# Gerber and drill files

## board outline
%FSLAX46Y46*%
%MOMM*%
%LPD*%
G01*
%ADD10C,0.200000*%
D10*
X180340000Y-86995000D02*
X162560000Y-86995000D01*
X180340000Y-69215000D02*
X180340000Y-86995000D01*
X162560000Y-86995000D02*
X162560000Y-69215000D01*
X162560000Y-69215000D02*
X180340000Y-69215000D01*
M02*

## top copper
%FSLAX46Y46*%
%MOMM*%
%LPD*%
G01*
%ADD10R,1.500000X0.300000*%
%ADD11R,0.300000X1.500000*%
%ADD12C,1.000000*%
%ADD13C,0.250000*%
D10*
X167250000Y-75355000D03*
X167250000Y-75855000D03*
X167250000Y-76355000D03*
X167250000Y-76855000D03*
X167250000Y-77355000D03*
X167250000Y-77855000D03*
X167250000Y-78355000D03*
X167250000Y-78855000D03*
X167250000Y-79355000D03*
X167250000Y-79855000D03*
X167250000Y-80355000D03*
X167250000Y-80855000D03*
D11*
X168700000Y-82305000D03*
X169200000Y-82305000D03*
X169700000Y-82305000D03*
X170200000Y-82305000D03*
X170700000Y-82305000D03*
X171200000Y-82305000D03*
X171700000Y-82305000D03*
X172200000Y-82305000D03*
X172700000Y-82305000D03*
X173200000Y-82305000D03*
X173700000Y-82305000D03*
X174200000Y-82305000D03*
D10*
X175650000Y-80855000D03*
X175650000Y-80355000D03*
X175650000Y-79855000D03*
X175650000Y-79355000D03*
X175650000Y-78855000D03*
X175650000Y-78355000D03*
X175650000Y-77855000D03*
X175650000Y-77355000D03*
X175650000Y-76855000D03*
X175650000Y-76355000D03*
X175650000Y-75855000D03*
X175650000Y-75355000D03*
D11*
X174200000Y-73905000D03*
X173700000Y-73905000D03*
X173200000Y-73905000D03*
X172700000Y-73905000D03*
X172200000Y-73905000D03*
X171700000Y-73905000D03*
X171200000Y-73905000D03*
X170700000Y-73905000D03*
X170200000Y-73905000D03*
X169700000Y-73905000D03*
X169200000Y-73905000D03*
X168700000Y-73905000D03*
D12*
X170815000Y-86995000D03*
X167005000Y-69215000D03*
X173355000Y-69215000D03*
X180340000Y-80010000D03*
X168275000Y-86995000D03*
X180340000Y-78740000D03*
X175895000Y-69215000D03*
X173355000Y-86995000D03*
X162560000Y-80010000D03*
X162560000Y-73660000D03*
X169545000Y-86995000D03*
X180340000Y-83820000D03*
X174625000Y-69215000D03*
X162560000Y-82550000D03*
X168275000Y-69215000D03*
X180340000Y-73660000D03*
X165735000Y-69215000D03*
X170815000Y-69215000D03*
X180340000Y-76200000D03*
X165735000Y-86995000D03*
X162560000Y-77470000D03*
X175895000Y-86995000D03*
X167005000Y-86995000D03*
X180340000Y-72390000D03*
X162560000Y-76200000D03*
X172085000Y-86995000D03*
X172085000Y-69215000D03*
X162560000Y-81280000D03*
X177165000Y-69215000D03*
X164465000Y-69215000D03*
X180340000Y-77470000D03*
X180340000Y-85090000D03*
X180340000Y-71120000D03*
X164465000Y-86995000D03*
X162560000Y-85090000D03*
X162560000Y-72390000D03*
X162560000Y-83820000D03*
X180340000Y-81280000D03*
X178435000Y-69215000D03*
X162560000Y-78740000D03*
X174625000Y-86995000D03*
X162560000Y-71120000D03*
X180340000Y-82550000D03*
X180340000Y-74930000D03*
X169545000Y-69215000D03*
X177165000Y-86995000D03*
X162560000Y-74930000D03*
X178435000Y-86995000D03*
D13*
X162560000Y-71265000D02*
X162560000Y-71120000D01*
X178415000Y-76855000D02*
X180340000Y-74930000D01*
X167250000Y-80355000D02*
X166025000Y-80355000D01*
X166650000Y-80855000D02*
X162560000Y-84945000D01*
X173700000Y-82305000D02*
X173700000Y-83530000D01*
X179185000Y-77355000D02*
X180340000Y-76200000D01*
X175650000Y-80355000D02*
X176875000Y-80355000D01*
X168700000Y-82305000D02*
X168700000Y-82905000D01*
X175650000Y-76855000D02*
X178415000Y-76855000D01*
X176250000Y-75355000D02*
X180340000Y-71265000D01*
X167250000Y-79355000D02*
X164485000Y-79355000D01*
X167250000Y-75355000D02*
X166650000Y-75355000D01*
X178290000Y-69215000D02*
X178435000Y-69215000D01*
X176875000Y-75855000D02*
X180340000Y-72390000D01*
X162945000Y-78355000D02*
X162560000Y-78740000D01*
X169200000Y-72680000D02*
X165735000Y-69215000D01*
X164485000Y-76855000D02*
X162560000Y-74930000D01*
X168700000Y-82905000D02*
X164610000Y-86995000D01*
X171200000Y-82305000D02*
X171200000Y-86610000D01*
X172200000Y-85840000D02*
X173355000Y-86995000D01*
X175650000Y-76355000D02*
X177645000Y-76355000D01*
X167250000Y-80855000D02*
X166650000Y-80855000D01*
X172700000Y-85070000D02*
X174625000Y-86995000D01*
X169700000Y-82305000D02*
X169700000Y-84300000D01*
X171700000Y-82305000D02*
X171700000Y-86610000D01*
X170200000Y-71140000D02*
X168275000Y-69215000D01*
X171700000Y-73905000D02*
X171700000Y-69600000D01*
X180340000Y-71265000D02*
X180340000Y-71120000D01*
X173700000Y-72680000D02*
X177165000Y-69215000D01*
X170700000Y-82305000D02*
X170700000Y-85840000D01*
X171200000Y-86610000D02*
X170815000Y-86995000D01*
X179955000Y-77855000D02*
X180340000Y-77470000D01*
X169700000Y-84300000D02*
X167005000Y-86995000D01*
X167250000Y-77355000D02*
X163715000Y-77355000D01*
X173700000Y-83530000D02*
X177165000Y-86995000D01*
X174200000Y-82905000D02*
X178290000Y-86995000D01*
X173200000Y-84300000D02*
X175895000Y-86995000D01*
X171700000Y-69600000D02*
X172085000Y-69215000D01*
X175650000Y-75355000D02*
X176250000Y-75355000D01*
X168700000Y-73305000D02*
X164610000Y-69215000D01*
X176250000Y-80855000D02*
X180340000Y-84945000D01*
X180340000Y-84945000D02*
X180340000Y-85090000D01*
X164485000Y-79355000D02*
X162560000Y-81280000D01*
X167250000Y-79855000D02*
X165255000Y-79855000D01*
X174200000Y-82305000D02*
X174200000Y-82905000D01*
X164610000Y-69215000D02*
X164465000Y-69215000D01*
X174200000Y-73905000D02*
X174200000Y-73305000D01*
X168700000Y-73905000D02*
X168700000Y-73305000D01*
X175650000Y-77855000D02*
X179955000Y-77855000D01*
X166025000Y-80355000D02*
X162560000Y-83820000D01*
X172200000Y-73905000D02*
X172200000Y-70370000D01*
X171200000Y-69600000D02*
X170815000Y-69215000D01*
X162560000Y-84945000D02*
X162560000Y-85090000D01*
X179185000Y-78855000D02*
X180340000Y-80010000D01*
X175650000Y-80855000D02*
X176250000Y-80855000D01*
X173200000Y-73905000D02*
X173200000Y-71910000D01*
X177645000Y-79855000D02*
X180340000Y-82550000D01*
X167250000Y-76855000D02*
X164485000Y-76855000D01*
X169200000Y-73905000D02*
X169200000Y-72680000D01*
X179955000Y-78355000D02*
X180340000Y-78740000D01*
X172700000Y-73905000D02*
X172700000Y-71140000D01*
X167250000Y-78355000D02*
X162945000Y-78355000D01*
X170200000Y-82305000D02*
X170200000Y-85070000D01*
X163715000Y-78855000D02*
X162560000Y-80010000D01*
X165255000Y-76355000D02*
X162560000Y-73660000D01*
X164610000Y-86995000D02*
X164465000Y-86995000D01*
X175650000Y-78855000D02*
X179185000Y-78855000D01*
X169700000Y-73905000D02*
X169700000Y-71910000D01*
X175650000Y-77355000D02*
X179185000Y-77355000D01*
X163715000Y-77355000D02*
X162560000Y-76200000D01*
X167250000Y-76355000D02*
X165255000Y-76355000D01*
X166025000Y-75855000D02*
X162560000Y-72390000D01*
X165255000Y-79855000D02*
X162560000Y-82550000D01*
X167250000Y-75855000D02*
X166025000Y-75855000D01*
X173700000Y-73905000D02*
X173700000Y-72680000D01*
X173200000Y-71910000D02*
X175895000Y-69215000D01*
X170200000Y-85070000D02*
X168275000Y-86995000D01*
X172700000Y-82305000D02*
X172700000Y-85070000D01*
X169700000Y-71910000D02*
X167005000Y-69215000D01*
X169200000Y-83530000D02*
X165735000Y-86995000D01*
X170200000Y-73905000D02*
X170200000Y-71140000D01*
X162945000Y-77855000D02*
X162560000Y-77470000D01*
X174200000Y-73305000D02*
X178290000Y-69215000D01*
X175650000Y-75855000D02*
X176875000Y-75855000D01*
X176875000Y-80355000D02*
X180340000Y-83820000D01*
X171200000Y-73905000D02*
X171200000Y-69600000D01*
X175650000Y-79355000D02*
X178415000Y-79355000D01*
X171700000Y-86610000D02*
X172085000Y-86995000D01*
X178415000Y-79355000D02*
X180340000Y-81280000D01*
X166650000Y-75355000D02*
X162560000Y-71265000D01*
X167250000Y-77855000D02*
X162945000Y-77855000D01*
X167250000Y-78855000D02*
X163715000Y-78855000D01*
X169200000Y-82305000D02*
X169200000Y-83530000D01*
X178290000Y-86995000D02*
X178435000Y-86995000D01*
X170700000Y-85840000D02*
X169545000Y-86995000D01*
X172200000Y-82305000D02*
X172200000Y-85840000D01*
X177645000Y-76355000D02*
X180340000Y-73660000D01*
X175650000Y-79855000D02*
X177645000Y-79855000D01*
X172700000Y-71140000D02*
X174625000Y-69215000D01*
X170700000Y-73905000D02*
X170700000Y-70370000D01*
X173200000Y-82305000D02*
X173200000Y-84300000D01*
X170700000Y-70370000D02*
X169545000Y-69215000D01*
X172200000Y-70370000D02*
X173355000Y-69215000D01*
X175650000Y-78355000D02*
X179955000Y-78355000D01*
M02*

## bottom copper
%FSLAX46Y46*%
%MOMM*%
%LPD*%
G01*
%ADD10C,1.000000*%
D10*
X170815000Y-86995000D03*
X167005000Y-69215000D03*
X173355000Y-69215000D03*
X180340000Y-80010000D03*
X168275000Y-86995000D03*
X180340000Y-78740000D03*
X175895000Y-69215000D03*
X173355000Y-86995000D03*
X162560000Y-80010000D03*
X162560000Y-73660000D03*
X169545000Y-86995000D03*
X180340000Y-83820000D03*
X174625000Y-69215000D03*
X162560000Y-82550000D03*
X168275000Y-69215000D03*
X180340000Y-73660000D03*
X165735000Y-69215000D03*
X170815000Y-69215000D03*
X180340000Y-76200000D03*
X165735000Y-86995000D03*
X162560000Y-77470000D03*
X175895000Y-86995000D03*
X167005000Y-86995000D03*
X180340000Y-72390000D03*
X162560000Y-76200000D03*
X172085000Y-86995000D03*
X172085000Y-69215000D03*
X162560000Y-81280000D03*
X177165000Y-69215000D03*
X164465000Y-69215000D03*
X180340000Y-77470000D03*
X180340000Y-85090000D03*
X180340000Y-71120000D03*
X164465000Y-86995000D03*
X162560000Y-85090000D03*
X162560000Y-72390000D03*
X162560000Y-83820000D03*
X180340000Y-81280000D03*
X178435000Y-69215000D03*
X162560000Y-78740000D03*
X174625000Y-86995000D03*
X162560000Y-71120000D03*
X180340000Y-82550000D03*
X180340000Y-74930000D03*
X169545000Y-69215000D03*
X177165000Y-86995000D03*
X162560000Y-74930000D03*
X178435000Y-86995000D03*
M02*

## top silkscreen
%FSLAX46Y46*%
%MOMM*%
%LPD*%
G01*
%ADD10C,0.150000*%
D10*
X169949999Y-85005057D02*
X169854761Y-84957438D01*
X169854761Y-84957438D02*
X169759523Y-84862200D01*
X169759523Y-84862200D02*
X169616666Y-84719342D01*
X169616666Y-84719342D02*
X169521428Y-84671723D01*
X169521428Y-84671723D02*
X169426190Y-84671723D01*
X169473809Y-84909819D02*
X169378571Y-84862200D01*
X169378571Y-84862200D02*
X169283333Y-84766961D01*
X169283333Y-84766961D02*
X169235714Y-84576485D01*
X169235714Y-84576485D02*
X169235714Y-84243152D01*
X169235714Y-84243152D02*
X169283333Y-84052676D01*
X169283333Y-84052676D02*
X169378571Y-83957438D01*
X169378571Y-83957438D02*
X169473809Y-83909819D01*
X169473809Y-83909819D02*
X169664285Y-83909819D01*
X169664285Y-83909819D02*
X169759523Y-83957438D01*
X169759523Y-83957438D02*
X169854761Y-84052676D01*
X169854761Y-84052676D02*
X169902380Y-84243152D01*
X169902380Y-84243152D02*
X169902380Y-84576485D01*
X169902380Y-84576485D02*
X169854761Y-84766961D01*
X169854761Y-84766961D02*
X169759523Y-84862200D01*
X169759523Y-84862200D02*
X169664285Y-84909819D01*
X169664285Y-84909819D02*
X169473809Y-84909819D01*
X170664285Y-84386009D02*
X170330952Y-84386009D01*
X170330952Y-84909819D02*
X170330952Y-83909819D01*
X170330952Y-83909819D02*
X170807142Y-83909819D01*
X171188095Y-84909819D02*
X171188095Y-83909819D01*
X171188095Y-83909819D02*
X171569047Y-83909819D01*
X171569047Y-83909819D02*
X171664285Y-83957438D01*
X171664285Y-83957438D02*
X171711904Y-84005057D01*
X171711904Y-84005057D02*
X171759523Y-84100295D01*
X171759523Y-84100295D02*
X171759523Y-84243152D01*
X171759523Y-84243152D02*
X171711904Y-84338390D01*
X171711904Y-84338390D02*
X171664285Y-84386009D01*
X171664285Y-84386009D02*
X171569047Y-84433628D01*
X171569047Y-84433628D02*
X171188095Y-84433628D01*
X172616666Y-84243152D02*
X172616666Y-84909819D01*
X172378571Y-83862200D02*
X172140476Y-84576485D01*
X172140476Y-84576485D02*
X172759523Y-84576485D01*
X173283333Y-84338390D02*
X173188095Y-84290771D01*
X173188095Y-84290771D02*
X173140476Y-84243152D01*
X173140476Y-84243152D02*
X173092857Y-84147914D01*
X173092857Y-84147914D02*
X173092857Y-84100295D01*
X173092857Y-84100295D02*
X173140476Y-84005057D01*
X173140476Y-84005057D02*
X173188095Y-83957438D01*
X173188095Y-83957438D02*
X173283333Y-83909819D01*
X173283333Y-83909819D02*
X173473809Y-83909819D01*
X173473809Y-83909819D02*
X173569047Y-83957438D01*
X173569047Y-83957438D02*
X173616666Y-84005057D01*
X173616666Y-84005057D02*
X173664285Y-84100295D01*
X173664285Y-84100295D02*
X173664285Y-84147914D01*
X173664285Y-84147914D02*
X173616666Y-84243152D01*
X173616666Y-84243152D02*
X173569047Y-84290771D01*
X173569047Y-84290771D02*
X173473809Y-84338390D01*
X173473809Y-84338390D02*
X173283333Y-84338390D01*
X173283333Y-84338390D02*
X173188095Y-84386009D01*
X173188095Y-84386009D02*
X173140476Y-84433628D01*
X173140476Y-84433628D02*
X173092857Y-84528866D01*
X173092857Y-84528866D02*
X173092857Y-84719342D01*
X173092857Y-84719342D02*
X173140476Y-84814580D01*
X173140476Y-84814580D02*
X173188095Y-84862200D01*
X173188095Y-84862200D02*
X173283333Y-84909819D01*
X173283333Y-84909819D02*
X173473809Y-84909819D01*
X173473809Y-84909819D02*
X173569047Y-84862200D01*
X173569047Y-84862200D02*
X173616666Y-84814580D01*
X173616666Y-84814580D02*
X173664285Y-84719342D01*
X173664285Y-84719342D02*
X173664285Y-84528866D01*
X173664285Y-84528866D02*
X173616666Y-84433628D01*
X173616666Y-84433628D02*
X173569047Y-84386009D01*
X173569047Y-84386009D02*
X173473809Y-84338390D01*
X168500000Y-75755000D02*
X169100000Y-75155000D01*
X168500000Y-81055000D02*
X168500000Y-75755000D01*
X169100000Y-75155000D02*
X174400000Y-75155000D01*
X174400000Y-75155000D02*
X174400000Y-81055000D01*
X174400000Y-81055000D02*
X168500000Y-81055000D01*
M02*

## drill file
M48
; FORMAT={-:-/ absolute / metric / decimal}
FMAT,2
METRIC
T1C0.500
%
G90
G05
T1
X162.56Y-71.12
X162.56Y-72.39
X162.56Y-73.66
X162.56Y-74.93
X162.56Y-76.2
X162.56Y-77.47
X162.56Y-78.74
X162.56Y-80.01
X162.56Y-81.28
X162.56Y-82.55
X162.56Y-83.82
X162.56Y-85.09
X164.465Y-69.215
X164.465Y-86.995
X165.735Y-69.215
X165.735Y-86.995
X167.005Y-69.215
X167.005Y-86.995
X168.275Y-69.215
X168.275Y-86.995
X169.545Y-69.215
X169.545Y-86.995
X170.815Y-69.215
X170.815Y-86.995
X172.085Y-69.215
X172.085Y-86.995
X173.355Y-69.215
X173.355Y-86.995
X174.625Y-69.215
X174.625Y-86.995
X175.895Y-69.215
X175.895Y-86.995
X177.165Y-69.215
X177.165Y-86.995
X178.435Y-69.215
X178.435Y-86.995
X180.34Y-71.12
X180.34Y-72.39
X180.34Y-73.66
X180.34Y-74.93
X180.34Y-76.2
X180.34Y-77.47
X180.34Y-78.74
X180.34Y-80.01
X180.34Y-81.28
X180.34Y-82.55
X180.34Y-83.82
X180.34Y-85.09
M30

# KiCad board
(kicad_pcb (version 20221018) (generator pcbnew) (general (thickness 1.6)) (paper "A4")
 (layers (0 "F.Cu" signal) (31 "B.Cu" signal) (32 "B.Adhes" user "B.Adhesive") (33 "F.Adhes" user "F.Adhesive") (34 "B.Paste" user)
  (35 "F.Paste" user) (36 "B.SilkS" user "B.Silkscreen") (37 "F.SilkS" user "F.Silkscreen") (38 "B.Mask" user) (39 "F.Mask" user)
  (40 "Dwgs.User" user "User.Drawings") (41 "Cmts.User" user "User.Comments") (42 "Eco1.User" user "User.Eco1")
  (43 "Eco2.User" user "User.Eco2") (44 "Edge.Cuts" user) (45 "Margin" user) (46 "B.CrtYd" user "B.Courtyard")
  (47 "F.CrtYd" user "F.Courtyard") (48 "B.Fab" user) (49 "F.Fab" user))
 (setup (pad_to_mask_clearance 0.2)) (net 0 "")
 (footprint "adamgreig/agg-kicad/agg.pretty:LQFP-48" (layer "F.Cu") (at 171.45 78.105)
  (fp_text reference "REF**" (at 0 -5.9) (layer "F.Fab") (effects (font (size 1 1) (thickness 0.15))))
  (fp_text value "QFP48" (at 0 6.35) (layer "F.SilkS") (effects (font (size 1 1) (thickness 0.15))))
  (fp_line (start -2.95 -2.35) (end -2.35 -2.95) (stroke (width 0.15) (type solid)) (layer "F.SilkS"))
  (fp_line (start -2.95 2.95) (end -2.95 -2.35) (stroke (width 0.15) (type solid)) (layer "F.SilkS"))
  (fp_line (start -2.35 -2.95) (end 2.95 -2.95) (stroke (width 0.15) (type solid)) (layer "F.SilkS"))
  (fp_line (start 2.95 -2.95) (end 2.95 2.95) (stroke (width 0.15) (type solid)) (layer "F.SilkS"))
  (fp_line (start 2.95 2.95) (end -2.95 2.95) (stroke (width 0.15) (type solid)) (layer "F.SilkS"))
  (pad "1" smd rect (at -4.2 -2.75) (size 1.5 0.3) (layers "F.Cu" "F.Paste" "F.Mask"))
  (pad "2" smd rect (at -4.2 -2.25) (size 1.5 0.3) (layers "F.Cu" "F.Paste" "F.Mask"))
  (pad "3" smd rect (at -4.2 -1.75) (size 1.5 0.3) (layers "F.Cu" "F.Paste" "F.Mask"))
  (pad "4" smd rect (at -4.2 -1.25) (size 1.5 0.3) (layers "F.Cu" "F.Paste" "F.Mask"))
  (pad "5" smd rect (at -4.2 -0.75) (size 1.5 0.3) (layers "F.Cu" "F.Paste" "F.Mask"))
  (pad "6" smd rect (at -4.2 -0.25) (size 1.5 0.3) (layers "F.Cu" "F.Paste" "F.Mask"))
  (pad "7" smd rect (at -4.2 0.25) (size 1.5 0.3) (layers "F.Cu" "F.Paste" "F.Mask"))
  (pad "8" smd rect (at -4.2 0.75) (size 1.5 0.3) (layers "F.Cu" "F.Paste" "F.Mask"))
  (pad "9" smd rect (at -4.2 1.25) (size 1.5 0.3) (layers "F.Cu" "F.Paste" "F.Mask"))
  (pad "10" smd rect (at -4.2 1.75) (size 1.5 0.3) (layers "F.Cu" "F.Paste" "F.Mask"))
  (pad "11" smd rect (at -4.2 2.25) (size 1.5 0.3) (layers "F.Cu" "F.Paste" "F.Mask"))
  (pad "12" smd rect (at -4.2 2.75) (size 1.5 0.3) (layers "F.Cu" "F.Paste" "F.Mask"))
  (pad "13" smd rect (at -2.75 4.2) (size 0.3 1.5) (layers "F.Cu" "F.Paste" "F.Mask"))
  (pad "14" smd rect (at -2.25 4.2) (size 0.3 1.5) (layers "F.Cu" "F.Paste" "F.Mask"))
  (pad "15" smd rect (at -1.75 4.2) (size 0.3 1.5) (layers "F.Cu" "F.Paste" "F.Mask"))
  (pad "16" smd rect (at -1.25 4.2) (size 0.3 1.5) (layers "F.Cu" "F.Paste" "F.Mask"))
  (pad "17" smd rect (at -0.75 4.2) (size 0.3 1.5) (layers "F.Cu" "F.Paste" "F.Mask"))
  (pad "18" smd rect (at -0.25 4.2) (size 0.3 1.5) (layers "F.Cu" "F.Paste" "F.Mask"))
  (pad "19" smd rect (at 0.25 4.2) (size 0.3 1.5) (layers "F.Cu" "F.Paste" "F.Mask"))
  (pad "20" smd rect (at 0.75 4.2) (size 0.3 1.5) (layers "F.Cu" "F.Paste" "F.Mask"))
  (pad "21" smd rect (at 1.25 4.2) (size 0.3 1.5) (layers "F.Cu" "F.Paste" "F.Mask"))
  (pad "22" smd rect (at 1.75 4.2) (size 0.3 1.5) (layers "F.Cu" "F.Paste" "F.Mask"))
  (pad "23" smd rect (at 2.25 4.2) (size 0.3 1.5) (layers "F.Cu" "F.Paste" "F.Mask"))
  (pad "24" smd rect (at 2.75 4.2) (size 0.3 1.5) (layers "F.Cu" "F.Paste" "F.Mask"))
  (pad "25" smd rect (at 4.2 2.75) (size 1.5 0.3) (layers "F.Cu" "F.Paste" "F.Mask"))
  (pad "26" smd rect (at 4.2 2.25) (size 1.5 0.3) (layers "F.Cu" "F.Paste" "F.Mask"))
  (pad "27" smd rect (at 4.2 1.75) (size 1.5 0.3) (layers "F.Cu" "F.Paste" "F.Mask"))
  (pad "28" smd rect (at 4.2 1.25) (size 1.5 0.3) (layers "F.Cu" "F.Paste" "F.Mask"))
  (pad "29" smd rect (at 4.2 0.75) (size 1.5 0.3) (layers "F.Cu" "F.Paste" "F.Mask"))
  (pad "30" smd rect (at 4.2 0.25) (size 1.5 0.3) (layers "F.Cu" "F.Paste" "F.Mask"))
  (pad "31" smd rect (at 4.2 -0.25) (size 1.5 0.3) (layers "F.Cu" "F.Paste" "F.Mask"))
  (pad "32" smd rect (at 4.2 -0.75) (size 1.5 0.3) (layers "F.Cu" "F.Paste" "F.Mask"))
  (pad "33" smd rect (at 4.2 -1.25) (size 1.5 0.3) (layers "F.Cu" "F.Paste" "F.Mask"))
  (pad "34" smd rect (at 4.2 -1.75) (size 1.5 0.3) (layers "F.Cu" "F.Paste" "F.Mask"))
  (pad "35" smd rect (at 4.2 -2.25) (size 1.5 0.3) (layers "F.Cu" "F.Paste" "F.Mask"))
  (pad "36" smd rect (at 4.2 -2.75) (size 1.5 0.3) (layers "F.Cu" "F.Paste" "F.Mask"))
  (pad "37" smd rect (at 2.75 -4.2) (size 0.3 1.5) (layers "F.Cu" "F.Paste" "F.Mask"))
  (pad "38" smd rect (at 2.25 -4.2) (size 0.3 1.5) (layers "F.Cu" "F.Paste" "F.Mask"))
  (pad "39" smd rect (at 1.75 -4.2) (size 0.3 1.5) (layers "F.Cu" "F.Paste" "F.Mask"))
  (pad "40" smd rect (at 1.25 -4.2) (size 0.3 1.5) (layers "F.Cu" "F.Paste" "F.Mask"))
  (pad "41" smd rect (at 0.75 -4.2) (size 0.3 1.5) (layers "F.Cu" "F.Paste" "F.Mask"))
  (pad "42" smd rect (at 0.25 -4.2) (size 0.3 1.5) (layers "F.Cu" "F.Paste" "F.Mask"))
  (pad "43" smd rect (at -0.25 -4.2) (size 0.3 1.5) (layers "F.Cu" "F.Paste" "F.Mask"))
  (pad "44" smd rect (at -0.75 -4.2) (size 0.3 1.5) (layers "F.Cu" "F.Paste" "F.Mask"))
  (pad "45" smd rect (at -1.25 -4.2) (size 0.3 1.5) (layers "F.Cu" "F.Paste" "F.Mask"))
  (pad "46" smd rect (at -1.75 -4.2) (size 0.3 1.5) (layers "F.Cu" "F.Paste" "F.Mask"))
  (pad "47" smd rect (at -2.25 -4.2) (size 0.3 1.5) (layers "F.Cu" "F.Paste" "F.Mask"))
  (pad "48" smd rect (at -2.75 -4.2) (size 0.3 1.5) (layers "F.Cu" "F.Paste" "F.Mask")))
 (gr_line (start 180.34 86.995) (end 162.56 86.995) (stroke (width 0.2) (type solid)) (layer "Edge.Cuts"))
 (gr_line (start 180.34 69.215) (end 180.34 86.995) (stroke (width 0.2) (type solid)) (layer "Edge.Cuts"))
 (gr_line (start 162.56 86.995) (end 162.56 69.215) (stroke (width 0.2) (type solid)) (layer "Edge.Cuts"))
 (gr_line (start 162.56 69.215) (end 180.34 69.215) (stroke (width 0.2) (type solid)) (layer "Edge.Cuts"))
 (segment (start 162.56 71.265) (end 162.56 71.12) (width 0.25) (layer "F.Cu") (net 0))
 (segment (start 178.415 76.855) (end 180.34 74.93) (width 0.25) (layer "F.Cu") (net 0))
 (segment (start 167.25 80.355) (end 166.025 80.355) (width 0.25) (layer "F.Cu") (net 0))
 (segment (start 166.65 80.855) (end 162.56 84.945) (width 0.25) (layer "F.Cu") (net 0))
 (segment (start 173.7 82.305) (end 173.7 83.53) (width 0.25) (layer "F.Cu") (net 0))
 (segment (start 179.185 77.355) (end 180.34 76.2) (width 0.25) (layer "F.Cu") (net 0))
 (segment (start 175.65 80.355) (end 176.875 80.355) (width 0.25) (layer "F.Cu") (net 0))
 (segment (start 168.7 82.305) (end 168.7 82.905) (width 0.25) (layer "F.Cu") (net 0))
 (segment (start 175.65 76.855) (end 178.415 76.855) (width 0.25) (layer "F.Cu") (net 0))
 (segment (start 176.25 75.355) (end 180.34 71.265) (width 0.25) (layer "F.Cu") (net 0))
 (segment (start 167.25 79.355) (end 164.485 79.355) (width 0.25) (layer "F.Cu") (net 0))
 (segment (start 167.25 75.355) (end 166.65 75.355) (width 0.25) (layer "F.Cu") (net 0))
 (segment (start 178.29 69.215) (end 178.435 69.215) (width 0.25) (layer "F.Cu") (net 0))
 (segment (start 176.875 75.855) (end 180.34 72.39) (width 0.25) (layer "F.Cu") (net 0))
 (segment (start 162.945 78.355) (end 162.56 78.74) (width 0.25) (layer "F.Cu") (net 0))
 (segment (start 169.2 72.68) (end 165.735 69.215) (width 0.25) (layer "F.Cu") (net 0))
 (segment (start 164.485 76.855) (end 162.56 74.93) (width 0.25) (layer "F.Cu") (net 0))
 (segment (start 168.7 82.905) (end 164.61 86.995) (width 0.25) (layer "F.Cu") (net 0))
 (segment (start 171.2 82.305) (end 171.2 86.61) (width 0.25) (layer "F.Cu") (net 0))
 (segment (start 172.2 85.84) (end 173.355 86.995) (width 0.25) (layer "F.Cu") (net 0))
 (segment (start 175.65 76.355) (end 177.645 76.355) (width 0.25) (layer "F.Cu") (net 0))
 (segment (start 167.25 80.855) (end 166.65 80.855) (width 0.25) (layer "F.Cu") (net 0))
 (segment (start 172.7 85.07) (end 174.625 86.995) (width 0.25) (layer "F.Cu") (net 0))
 (segment (start 169.7 82.305) (end 169.7 84.3) (width 0.25) (layer "F.Cu") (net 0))
 (segment (start 171.7 82.305) (end 171.7 86.61) (width 0.25) (layer "F.Cu") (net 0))
 (segment (start 170.2 71.14) (end 168.275 69.215) (width 0.25) (layer "F.Cu") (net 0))
 (segment (start 171.7 73.905) (end 171.7 69.6) (width 0.25) (layer "F.Cu") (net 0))
 (segment (start 180.34 71.265) (end 180.34 71.12) (width 0.25) (layer "F.Cu") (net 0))
 (segment (start 173.7 72.68) (end 177.165 69.215) (width 0.25) (layer "F.Cu") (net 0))
 (segment (start 170.7 82.305) (end 170.7 85.84) (width 0.25) (layer "F.Cu") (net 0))
 (segment (start 171.2 86.61) (end 170.815 86.995) (width 0.25) (layer "F.Cu") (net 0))
 (segment (start 179.955 77.855) (end 180.34 77.47) (width 0.25) (layer "F.Cu") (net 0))
 (segment (start 169.7 84.3) (end 167.005 86.995) (width 0.25) (layer "F.Cu") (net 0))
 (segment (start 167.25 77.355) (end 163.715 77.355) (width 0.25) (layer "F.Cu") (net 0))
 (segment (start 173.7 83.53) (end 177.165 86.995) (width 0.25) (layer "F.Cu") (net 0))
 (segment (start 174.2 82.905) (end 178.29 86.995) (width 0.25) (layer "F.Cu") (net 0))
 (segment (start 173.2 84.3) (end 175.895 86.995) (width 0.25) (layer "F.Cu") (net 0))
 (segment (start 171.7 69.6) (end 172.085 69.215) (width 0.25) (layer "F.Cu") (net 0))
 (segment (start 175.65 75.355) (end 176.25 75.355) (width 0.25) (layer "F.Cu") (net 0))
 (segment (start 168.7 73.305) (end 164.61 69.215) (width 0.25) (layer "F.Cu") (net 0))
 (segment (start 176.25 80.855) (end 180.34 84.945) (width 0.25) (layer "F.Cu") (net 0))
 (segment (start 180.34 84.945) (end 180.34 85.09) (width 0.25) (layer "F.Cu") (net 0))
 (segment (start 164.485 79.355) (end 162.56 81.28) (width 0.25) (layer "F.Cu") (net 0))
 (segment (start 167.25 79.855) (end 165.255 79.855) (width 0.25) (layer "F.Cu") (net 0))
 (segment (start 174.2 82.305) (end 174.2 82.905) (width 0.25) (layer "F.Cu") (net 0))
 (segment (start 164.61 69.215) (end 164.465 69.215) (width 0.25) (layer "F.Cu") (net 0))
 (segment (start 174.2 73.905) (end 174.2 73.305) (width 0.25) (layer "F.Cu") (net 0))
 (segment (start 168.7 73.905) (end 168.7 73.305) (width 0.25) (layer "F.Cu") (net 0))
 (segment (start 175.65 77.855) (end 179.955 77.855) (width 0.25) (layer "F.Cu") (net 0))
 (segment (start 166.025 80.355) (end 162.56 83.82) (width 0.25) (layer "F.Cu") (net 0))
 (segment (start 172.2 73.905) (end 172.2 70.37) (width 0.25) (layer "F.Cu") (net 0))
 (segment (start 171.2 69.6) (end 170.815 69.215) (width 0.25) (layer "F.Cu") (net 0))
 (segment (start 162.56 84.945) (end 162.56 85.09) (width 0.25) (layer "F.Cu") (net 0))
 (segment (start 179.185 78.855) (end 180.34 80.01) (width 0.25) (layer "F.Cu") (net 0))
 (segment (start 175.65 80.855) (end 176.25 80.855) (width 0.25) (layer "F.Cu") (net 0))
 (segment (start 173.2 73.905) (end 173.2 71.91) (width 0.25) (layer "F.Cu") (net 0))
 (segment (start 177.645 79.855) (end 180.34 82.55) (width 0.25) (layer "F.Cu") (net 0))
 (segment (start 167.25 76.855) (end 164.485 76.855) (width 0.25) (layer "F.Cu") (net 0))
 (segment (start 169.2 73.905) (end 169.2 72.68) (width 0.25) (layer "F.Cu") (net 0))
 (segment (start 179.955 78.355) (end 180.34 78.74) (width 0.25) (layer "F.Cu") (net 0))
 (segment (start 172.7 73.905) (end 172.7 71.14) (width 0.25) (layer "F.Cu") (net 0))
 (segment (start 167.25 78.355) (end 162.945 78.355) (width 0.25) (layer "F.Cu") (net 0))
 (segment (start 170.2 82.305) (end 170.2 85.07) (width 0.25) (layer "F.Cu") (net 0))
 (segment (start 163.715 78.855) (end 162.56 80.01) (width 0.25) (layer "F.Cu") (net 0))
 (segment (start 165.255 76.355) (end 162.56 73.66) (width 0.25) (layer "F.Cu") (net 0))
 (segment (start 164.61 86.995) (end 164.465 86.995) (width 0.25) (layer "F.Cu") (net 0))
 (segment (start 175.65 78.855) (end 179.185 78.855) (width 0.25) (layer "F.Cu") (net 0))
 (segment (start 169.7 73.905) (end 169.7 71.91) (width 0.25) (layer "F.Cu") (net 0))
 (segment (start 175.65 77.355) (end 179.185 77.355) (width 0.25) (layer "F.Cu") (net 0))
 (segment (start 163.715 77.355) (end 162.56 76.2) (width 0.25) (layer "F.Cu") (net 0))
 (segment (start 167.25 76.355) (end 165.255 76.355) (width 0.25) (layer "F.Cu") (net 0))
 (segment (start 166.025 75.855) (end 162.56 72.39) (width 0.25) (layer "F.Cu") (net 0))
 (segment (start 165.255 79.855) (end 162.56 82.55) (width 0.25) (layer "F.Cu") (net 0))
 (segment (start 167.25 75.855) (end 166.025 75.855) (width 0.25) (layer "F.Cu") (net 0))
 (segment (start 173.7 73.905) (end 173.7 72.68) (width 0.25) (layer "F.Cu") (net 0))
 (segment (start 173.2 71.91) (end 175.895 69.215) (width 0.25) (layer "F.Cu") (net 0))
 (segment (start 170.2 85.07) (end 168.275 86.995) (width 0.25) (layer "F.Cu") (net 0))
 (segment (start 172.7 82.305) (end 172.7 85.07) (width 0.25) (layer "F.Cu") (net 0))
 (segment (start 169.7 71.91) (end 167.005 69.215) (width 0.25) (layer "F.Cu") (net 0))
 (segment (start 169.2 83.53) (end 165.735 86.995) (width 0.25) (layer "F.Cu") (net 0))
 (segment (start 170.2 73.905) (end 170.2 71.14) (width 0.25) (layer "F.Cu") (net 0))
 (segment (start 162.945 77.855) (end 162.56 77.47) (width 0.25) (layer "F.Cu") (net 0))
 (segment (start 174.2 73.305) (end 178.29 69.215) (width 0.25) (layer "F.Cu") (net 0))
 (segment (start 175.65 75.855) (end 176.875 75.855) (width 0.25) (layer "F.Cu") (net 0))
 (segment (start 176.875 80.355) (end 180.34 83.82) (width 0.25) (layer "F.Cu") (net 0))
 (segment (start 171.2 73.905) (end 171.2 69.6) (width 0.25) (layer "F.Cu") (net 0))
 (segment (start 175.65 79.355) (end 178.415 79.355) (width 0.25) (layer "F.Cu") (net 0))
 (segment (start 171.7 86.61) (end 172.085 86.995) (width 0.25) (layer "F.Cu") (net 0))
 (segment (start 178.415 79.355) (end 180.34 81.28) (width 0.25) (layer "F.Cu") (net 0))
 (segment (start 166.65 75.355) (end 162.56 71.265) (width 0.25) (layer "F.Cu") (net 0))
 (segment (start 167.25 77.855) (end 162.945 77.855) (width 0.25) (layer "F.Cu") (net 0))
 (segment (start 167.25 78.855) (end 163.715 78.855) (width 0.25) (layer "F.Cu") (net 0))
 (segment (start 169.2 82.305) (end 169.2 83.53) (width 0.25) (layer "F.Cu") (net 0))
 (segment (start 178.29 86.995) (end 178.435 86.995) (width 0.25) (layer "F.Cu") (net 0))
 (segment (start 170.7 85.84) (end 169.545 86.995) (width 0.25) (layer "F.Cu") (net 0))
 (segment (start 172.2 82.305) (end 172.2 85.84) (width 0.25) (layer "F.Cu") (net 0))
 (segment (start 177.645 76.355) (end 180.34 73.66) (width 0.25) (layer "F.Cu") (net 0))
 (segment (start 175.65 79.855) (end 177.645 79.855) (width 0.25) (layer "F.Cu") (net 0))
 (segment (start 172.7 71.14) (end 174.625 69.215) (width 0.25) (layer "F.Cu") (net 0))
 (segment (start 170.7 73.905) (end 170.7 70.37) (width 0.25) (layer "F.Cu") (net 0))
 (segment (start 173.2 82.305) (end 173.2 84.3) (width 0.25) (layer "F.Cu") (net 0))
 (segment (start 170.7 70.37) (end 169.545 69.215) (width 0.25) (layer "F.Cu") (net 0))
 (segment (start 172.2 70.37) (end 173.355 69.215) (width 0.25) (layer "F.Cu") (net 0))
 (segment (start 175.65 78.355) (end 179.955 78.355) (width 0.25) (layer "F.Cu") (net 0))
 (via (at 170.815 86.995) (size 1) (drill 0.5) (layers "F.Cu" "B.Cu") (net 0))
 (via (at 167.005 69.215) (size 1) (drill 0.5) (layers "F.Cu" "B.Cu") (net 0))
 (via (at 173.355 69.215) (size 1) (drill 0.5) (layers "F.Cu" "B.Cu") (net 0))
 (via (at 180.34 80.01) (size 1) (drill 0.5) (layers "F.Cu" "B.Cu") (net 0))
 (via (at 168.275 86.995) (size 1) (drill 0.5) (layers "F.Cu" "B.Cu") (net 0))
 (via (at 180.34 78.74) (size 1) (drill 0.5) (layers "F.Cu" "B.Cu") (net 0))
 (via (at 175.895 69.215) (size 1) (drill 0.5) (layers "F.Cu" "B.Cu") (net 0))
 (via (at 173.355 86.995) (size 1) (drill 0.5) (layers "F.Cu" "B.Cu") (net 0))
 (via (at 162.56 80.01) (size 1) (drill 0.5) (layers "F.Cu" "B.Cu") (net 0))
 (via (at 162.56 73.66) (size 1) (drill 0.5) (layers "F.Cu" "B.Cu") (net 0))
 (via (at 169.545 86.995) (size 1) (drill 0.5) (layers "F.Cu" "B.Cu") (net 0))
 (via (at 180.34 83.82) (size 1) (drill 0.5) (layers "F.Cu" "B.Cu") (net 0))
 (via (at 174.625 69.215) (size 1) (drill 0.5) (layers "F.Cu" "B.Cu") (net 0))
 (via (at 162.56 82.55) (size 1) (drill 0.5) (layers "F.Cu" "B.Cu") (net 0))
 (via (at 168.275 69.215) (size 1) (drill 0.5) (layers "F.Cu" "B.Cu") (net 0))
 (via (at 180.34 73.66) (size 1) (drill 0.5) (layers "F.Cu" "B.Cu") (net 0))
 (via (at 165.735 69.215) (size 1) (drill 0.5) (layers "F.Cu" "B.Cu") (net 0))
 (via (at 170.815 69.215) (size 1) (drill 0.5) (layers "F.Cu" "B.Cu") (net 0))
 (via (at 180.34 76.2) (size 1) (drill 0.5) (layers "F.Cu" "B.Cu") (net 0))
 (via (at 165.735 86.995) (size 1) (drill 0.5) (layers "F.Cu" "B.Cu") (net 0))
 (via (at 162.56 77.47) (size 1) (drill 0.5) (layers "F.Cu" "B.Cu") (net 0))
 (via (at 175.895 86.995) (size 1) (drill 0.5) (layers "F.Cu" "B.Cu") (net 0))
 (via (at 167.005 86.995) (size 1) (drill 0.5) (layers "F.Cu" "B.Cu") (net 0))
 (via (at 180.34 72.39) (size 1) (drill 0.5) (layers "F.Cu" "B.Cu") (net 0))
 (via (at 162.56 76.2) (size 1) (drill 0.5) (layers "F.Cu" "B.Cu") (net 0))
 (via (at 172.085 86.995) (size 1) (drill 0.5) (layers "F.Cu" "B.Cu") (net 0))
 (via (at 172.085 69.215) (size 1) (drill 0.5) (layers "F.Cu" "B.Cu") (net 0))
 (via (at 162.56 81.28) (size 1) (drill 0.5) (layers "F.Cu" "B.Cu") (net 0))
 (via (at 177.165 69.215) (size 1) (drill 0.5) (layers "F.Cu" "B.Cu") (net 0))
 (via (at 164.465 69.215) (size 1) (drill 0.5) (layers "F.Cu" "B.Cu") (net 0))
 (via (at 180.34 77.47) (size 1) (drill 0.5) (layers "F.Cu" "B.Cu") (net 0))
 (via (at 180.34 85.09) (size 1) (drill 0.5) (layers "F.Cu" "B.Cu") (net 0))
 (via (at 180.34 71.12) (size 1) (drill 0.5) (layers "F.Cu" "B.Cu") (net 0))
 (via (at 164.465 86.995) (size 1) (drill 0.5) (layers "F.Cu" "B.Cu") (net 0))
 (via (at 162.56 85.09) (size 1) (drill 0.5) (layers "F.Cu" "B.Cu") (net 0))
 (via (at 162.56 72.39) (size 1) (drill 0.5) (layers "F.Cu" "B.Cu") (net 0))
 (via (at 162.56 83.82) (size 1) (drill 0.5) (layers "F.Cu" "B.Cu") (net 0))
 (via (at 180.34 81.28) (size 1) (drill 0.5) (layers "F.Cu" "B.Cu") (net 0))
 (via (at 178.435 69.215) (size 1) (drill 0.5) (layers "F.Cu" "B.Cu") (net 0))
 (via (at 162.56 78.74) (size 1) (drill 0.5) (layers "F.Cu" "B.Cu") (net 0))
 (via (at 174.625 86.995) (size 1) (drill 0.5) (layers "F.Cu" "B.Cu") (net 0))
 (via (at 162.56 71.12) (size 1) (drill 0.5) (layers "F.Cu" "B.Cu") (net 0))
 (via (at 180.34 82.55) (size 1) (drill 0.5) (layers "F.Cu" "B.Cu") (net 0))
 (via (at 180.34 74.93) (size 1) (drill 0.5) (layers "F.Cu" "B.Cu") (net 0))
 (via (at 169.545 69.215) (size 1) (drill 0.5) (layers "F.Cu" "B.Cu") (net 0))
 (via (at 177.165 86.995) (size 1) (drill 0.5) (layers "F.Cu" "B.Cu") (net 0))
 (via (at 162.56 74.93) (size 1) (drill 0.5) (layers "F.Cu" "B.Cu") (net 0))
 (via (at 178.435 86.995) (size 1) (drill 0.5) (layers "F.Cu" "B.Cu") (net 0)))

